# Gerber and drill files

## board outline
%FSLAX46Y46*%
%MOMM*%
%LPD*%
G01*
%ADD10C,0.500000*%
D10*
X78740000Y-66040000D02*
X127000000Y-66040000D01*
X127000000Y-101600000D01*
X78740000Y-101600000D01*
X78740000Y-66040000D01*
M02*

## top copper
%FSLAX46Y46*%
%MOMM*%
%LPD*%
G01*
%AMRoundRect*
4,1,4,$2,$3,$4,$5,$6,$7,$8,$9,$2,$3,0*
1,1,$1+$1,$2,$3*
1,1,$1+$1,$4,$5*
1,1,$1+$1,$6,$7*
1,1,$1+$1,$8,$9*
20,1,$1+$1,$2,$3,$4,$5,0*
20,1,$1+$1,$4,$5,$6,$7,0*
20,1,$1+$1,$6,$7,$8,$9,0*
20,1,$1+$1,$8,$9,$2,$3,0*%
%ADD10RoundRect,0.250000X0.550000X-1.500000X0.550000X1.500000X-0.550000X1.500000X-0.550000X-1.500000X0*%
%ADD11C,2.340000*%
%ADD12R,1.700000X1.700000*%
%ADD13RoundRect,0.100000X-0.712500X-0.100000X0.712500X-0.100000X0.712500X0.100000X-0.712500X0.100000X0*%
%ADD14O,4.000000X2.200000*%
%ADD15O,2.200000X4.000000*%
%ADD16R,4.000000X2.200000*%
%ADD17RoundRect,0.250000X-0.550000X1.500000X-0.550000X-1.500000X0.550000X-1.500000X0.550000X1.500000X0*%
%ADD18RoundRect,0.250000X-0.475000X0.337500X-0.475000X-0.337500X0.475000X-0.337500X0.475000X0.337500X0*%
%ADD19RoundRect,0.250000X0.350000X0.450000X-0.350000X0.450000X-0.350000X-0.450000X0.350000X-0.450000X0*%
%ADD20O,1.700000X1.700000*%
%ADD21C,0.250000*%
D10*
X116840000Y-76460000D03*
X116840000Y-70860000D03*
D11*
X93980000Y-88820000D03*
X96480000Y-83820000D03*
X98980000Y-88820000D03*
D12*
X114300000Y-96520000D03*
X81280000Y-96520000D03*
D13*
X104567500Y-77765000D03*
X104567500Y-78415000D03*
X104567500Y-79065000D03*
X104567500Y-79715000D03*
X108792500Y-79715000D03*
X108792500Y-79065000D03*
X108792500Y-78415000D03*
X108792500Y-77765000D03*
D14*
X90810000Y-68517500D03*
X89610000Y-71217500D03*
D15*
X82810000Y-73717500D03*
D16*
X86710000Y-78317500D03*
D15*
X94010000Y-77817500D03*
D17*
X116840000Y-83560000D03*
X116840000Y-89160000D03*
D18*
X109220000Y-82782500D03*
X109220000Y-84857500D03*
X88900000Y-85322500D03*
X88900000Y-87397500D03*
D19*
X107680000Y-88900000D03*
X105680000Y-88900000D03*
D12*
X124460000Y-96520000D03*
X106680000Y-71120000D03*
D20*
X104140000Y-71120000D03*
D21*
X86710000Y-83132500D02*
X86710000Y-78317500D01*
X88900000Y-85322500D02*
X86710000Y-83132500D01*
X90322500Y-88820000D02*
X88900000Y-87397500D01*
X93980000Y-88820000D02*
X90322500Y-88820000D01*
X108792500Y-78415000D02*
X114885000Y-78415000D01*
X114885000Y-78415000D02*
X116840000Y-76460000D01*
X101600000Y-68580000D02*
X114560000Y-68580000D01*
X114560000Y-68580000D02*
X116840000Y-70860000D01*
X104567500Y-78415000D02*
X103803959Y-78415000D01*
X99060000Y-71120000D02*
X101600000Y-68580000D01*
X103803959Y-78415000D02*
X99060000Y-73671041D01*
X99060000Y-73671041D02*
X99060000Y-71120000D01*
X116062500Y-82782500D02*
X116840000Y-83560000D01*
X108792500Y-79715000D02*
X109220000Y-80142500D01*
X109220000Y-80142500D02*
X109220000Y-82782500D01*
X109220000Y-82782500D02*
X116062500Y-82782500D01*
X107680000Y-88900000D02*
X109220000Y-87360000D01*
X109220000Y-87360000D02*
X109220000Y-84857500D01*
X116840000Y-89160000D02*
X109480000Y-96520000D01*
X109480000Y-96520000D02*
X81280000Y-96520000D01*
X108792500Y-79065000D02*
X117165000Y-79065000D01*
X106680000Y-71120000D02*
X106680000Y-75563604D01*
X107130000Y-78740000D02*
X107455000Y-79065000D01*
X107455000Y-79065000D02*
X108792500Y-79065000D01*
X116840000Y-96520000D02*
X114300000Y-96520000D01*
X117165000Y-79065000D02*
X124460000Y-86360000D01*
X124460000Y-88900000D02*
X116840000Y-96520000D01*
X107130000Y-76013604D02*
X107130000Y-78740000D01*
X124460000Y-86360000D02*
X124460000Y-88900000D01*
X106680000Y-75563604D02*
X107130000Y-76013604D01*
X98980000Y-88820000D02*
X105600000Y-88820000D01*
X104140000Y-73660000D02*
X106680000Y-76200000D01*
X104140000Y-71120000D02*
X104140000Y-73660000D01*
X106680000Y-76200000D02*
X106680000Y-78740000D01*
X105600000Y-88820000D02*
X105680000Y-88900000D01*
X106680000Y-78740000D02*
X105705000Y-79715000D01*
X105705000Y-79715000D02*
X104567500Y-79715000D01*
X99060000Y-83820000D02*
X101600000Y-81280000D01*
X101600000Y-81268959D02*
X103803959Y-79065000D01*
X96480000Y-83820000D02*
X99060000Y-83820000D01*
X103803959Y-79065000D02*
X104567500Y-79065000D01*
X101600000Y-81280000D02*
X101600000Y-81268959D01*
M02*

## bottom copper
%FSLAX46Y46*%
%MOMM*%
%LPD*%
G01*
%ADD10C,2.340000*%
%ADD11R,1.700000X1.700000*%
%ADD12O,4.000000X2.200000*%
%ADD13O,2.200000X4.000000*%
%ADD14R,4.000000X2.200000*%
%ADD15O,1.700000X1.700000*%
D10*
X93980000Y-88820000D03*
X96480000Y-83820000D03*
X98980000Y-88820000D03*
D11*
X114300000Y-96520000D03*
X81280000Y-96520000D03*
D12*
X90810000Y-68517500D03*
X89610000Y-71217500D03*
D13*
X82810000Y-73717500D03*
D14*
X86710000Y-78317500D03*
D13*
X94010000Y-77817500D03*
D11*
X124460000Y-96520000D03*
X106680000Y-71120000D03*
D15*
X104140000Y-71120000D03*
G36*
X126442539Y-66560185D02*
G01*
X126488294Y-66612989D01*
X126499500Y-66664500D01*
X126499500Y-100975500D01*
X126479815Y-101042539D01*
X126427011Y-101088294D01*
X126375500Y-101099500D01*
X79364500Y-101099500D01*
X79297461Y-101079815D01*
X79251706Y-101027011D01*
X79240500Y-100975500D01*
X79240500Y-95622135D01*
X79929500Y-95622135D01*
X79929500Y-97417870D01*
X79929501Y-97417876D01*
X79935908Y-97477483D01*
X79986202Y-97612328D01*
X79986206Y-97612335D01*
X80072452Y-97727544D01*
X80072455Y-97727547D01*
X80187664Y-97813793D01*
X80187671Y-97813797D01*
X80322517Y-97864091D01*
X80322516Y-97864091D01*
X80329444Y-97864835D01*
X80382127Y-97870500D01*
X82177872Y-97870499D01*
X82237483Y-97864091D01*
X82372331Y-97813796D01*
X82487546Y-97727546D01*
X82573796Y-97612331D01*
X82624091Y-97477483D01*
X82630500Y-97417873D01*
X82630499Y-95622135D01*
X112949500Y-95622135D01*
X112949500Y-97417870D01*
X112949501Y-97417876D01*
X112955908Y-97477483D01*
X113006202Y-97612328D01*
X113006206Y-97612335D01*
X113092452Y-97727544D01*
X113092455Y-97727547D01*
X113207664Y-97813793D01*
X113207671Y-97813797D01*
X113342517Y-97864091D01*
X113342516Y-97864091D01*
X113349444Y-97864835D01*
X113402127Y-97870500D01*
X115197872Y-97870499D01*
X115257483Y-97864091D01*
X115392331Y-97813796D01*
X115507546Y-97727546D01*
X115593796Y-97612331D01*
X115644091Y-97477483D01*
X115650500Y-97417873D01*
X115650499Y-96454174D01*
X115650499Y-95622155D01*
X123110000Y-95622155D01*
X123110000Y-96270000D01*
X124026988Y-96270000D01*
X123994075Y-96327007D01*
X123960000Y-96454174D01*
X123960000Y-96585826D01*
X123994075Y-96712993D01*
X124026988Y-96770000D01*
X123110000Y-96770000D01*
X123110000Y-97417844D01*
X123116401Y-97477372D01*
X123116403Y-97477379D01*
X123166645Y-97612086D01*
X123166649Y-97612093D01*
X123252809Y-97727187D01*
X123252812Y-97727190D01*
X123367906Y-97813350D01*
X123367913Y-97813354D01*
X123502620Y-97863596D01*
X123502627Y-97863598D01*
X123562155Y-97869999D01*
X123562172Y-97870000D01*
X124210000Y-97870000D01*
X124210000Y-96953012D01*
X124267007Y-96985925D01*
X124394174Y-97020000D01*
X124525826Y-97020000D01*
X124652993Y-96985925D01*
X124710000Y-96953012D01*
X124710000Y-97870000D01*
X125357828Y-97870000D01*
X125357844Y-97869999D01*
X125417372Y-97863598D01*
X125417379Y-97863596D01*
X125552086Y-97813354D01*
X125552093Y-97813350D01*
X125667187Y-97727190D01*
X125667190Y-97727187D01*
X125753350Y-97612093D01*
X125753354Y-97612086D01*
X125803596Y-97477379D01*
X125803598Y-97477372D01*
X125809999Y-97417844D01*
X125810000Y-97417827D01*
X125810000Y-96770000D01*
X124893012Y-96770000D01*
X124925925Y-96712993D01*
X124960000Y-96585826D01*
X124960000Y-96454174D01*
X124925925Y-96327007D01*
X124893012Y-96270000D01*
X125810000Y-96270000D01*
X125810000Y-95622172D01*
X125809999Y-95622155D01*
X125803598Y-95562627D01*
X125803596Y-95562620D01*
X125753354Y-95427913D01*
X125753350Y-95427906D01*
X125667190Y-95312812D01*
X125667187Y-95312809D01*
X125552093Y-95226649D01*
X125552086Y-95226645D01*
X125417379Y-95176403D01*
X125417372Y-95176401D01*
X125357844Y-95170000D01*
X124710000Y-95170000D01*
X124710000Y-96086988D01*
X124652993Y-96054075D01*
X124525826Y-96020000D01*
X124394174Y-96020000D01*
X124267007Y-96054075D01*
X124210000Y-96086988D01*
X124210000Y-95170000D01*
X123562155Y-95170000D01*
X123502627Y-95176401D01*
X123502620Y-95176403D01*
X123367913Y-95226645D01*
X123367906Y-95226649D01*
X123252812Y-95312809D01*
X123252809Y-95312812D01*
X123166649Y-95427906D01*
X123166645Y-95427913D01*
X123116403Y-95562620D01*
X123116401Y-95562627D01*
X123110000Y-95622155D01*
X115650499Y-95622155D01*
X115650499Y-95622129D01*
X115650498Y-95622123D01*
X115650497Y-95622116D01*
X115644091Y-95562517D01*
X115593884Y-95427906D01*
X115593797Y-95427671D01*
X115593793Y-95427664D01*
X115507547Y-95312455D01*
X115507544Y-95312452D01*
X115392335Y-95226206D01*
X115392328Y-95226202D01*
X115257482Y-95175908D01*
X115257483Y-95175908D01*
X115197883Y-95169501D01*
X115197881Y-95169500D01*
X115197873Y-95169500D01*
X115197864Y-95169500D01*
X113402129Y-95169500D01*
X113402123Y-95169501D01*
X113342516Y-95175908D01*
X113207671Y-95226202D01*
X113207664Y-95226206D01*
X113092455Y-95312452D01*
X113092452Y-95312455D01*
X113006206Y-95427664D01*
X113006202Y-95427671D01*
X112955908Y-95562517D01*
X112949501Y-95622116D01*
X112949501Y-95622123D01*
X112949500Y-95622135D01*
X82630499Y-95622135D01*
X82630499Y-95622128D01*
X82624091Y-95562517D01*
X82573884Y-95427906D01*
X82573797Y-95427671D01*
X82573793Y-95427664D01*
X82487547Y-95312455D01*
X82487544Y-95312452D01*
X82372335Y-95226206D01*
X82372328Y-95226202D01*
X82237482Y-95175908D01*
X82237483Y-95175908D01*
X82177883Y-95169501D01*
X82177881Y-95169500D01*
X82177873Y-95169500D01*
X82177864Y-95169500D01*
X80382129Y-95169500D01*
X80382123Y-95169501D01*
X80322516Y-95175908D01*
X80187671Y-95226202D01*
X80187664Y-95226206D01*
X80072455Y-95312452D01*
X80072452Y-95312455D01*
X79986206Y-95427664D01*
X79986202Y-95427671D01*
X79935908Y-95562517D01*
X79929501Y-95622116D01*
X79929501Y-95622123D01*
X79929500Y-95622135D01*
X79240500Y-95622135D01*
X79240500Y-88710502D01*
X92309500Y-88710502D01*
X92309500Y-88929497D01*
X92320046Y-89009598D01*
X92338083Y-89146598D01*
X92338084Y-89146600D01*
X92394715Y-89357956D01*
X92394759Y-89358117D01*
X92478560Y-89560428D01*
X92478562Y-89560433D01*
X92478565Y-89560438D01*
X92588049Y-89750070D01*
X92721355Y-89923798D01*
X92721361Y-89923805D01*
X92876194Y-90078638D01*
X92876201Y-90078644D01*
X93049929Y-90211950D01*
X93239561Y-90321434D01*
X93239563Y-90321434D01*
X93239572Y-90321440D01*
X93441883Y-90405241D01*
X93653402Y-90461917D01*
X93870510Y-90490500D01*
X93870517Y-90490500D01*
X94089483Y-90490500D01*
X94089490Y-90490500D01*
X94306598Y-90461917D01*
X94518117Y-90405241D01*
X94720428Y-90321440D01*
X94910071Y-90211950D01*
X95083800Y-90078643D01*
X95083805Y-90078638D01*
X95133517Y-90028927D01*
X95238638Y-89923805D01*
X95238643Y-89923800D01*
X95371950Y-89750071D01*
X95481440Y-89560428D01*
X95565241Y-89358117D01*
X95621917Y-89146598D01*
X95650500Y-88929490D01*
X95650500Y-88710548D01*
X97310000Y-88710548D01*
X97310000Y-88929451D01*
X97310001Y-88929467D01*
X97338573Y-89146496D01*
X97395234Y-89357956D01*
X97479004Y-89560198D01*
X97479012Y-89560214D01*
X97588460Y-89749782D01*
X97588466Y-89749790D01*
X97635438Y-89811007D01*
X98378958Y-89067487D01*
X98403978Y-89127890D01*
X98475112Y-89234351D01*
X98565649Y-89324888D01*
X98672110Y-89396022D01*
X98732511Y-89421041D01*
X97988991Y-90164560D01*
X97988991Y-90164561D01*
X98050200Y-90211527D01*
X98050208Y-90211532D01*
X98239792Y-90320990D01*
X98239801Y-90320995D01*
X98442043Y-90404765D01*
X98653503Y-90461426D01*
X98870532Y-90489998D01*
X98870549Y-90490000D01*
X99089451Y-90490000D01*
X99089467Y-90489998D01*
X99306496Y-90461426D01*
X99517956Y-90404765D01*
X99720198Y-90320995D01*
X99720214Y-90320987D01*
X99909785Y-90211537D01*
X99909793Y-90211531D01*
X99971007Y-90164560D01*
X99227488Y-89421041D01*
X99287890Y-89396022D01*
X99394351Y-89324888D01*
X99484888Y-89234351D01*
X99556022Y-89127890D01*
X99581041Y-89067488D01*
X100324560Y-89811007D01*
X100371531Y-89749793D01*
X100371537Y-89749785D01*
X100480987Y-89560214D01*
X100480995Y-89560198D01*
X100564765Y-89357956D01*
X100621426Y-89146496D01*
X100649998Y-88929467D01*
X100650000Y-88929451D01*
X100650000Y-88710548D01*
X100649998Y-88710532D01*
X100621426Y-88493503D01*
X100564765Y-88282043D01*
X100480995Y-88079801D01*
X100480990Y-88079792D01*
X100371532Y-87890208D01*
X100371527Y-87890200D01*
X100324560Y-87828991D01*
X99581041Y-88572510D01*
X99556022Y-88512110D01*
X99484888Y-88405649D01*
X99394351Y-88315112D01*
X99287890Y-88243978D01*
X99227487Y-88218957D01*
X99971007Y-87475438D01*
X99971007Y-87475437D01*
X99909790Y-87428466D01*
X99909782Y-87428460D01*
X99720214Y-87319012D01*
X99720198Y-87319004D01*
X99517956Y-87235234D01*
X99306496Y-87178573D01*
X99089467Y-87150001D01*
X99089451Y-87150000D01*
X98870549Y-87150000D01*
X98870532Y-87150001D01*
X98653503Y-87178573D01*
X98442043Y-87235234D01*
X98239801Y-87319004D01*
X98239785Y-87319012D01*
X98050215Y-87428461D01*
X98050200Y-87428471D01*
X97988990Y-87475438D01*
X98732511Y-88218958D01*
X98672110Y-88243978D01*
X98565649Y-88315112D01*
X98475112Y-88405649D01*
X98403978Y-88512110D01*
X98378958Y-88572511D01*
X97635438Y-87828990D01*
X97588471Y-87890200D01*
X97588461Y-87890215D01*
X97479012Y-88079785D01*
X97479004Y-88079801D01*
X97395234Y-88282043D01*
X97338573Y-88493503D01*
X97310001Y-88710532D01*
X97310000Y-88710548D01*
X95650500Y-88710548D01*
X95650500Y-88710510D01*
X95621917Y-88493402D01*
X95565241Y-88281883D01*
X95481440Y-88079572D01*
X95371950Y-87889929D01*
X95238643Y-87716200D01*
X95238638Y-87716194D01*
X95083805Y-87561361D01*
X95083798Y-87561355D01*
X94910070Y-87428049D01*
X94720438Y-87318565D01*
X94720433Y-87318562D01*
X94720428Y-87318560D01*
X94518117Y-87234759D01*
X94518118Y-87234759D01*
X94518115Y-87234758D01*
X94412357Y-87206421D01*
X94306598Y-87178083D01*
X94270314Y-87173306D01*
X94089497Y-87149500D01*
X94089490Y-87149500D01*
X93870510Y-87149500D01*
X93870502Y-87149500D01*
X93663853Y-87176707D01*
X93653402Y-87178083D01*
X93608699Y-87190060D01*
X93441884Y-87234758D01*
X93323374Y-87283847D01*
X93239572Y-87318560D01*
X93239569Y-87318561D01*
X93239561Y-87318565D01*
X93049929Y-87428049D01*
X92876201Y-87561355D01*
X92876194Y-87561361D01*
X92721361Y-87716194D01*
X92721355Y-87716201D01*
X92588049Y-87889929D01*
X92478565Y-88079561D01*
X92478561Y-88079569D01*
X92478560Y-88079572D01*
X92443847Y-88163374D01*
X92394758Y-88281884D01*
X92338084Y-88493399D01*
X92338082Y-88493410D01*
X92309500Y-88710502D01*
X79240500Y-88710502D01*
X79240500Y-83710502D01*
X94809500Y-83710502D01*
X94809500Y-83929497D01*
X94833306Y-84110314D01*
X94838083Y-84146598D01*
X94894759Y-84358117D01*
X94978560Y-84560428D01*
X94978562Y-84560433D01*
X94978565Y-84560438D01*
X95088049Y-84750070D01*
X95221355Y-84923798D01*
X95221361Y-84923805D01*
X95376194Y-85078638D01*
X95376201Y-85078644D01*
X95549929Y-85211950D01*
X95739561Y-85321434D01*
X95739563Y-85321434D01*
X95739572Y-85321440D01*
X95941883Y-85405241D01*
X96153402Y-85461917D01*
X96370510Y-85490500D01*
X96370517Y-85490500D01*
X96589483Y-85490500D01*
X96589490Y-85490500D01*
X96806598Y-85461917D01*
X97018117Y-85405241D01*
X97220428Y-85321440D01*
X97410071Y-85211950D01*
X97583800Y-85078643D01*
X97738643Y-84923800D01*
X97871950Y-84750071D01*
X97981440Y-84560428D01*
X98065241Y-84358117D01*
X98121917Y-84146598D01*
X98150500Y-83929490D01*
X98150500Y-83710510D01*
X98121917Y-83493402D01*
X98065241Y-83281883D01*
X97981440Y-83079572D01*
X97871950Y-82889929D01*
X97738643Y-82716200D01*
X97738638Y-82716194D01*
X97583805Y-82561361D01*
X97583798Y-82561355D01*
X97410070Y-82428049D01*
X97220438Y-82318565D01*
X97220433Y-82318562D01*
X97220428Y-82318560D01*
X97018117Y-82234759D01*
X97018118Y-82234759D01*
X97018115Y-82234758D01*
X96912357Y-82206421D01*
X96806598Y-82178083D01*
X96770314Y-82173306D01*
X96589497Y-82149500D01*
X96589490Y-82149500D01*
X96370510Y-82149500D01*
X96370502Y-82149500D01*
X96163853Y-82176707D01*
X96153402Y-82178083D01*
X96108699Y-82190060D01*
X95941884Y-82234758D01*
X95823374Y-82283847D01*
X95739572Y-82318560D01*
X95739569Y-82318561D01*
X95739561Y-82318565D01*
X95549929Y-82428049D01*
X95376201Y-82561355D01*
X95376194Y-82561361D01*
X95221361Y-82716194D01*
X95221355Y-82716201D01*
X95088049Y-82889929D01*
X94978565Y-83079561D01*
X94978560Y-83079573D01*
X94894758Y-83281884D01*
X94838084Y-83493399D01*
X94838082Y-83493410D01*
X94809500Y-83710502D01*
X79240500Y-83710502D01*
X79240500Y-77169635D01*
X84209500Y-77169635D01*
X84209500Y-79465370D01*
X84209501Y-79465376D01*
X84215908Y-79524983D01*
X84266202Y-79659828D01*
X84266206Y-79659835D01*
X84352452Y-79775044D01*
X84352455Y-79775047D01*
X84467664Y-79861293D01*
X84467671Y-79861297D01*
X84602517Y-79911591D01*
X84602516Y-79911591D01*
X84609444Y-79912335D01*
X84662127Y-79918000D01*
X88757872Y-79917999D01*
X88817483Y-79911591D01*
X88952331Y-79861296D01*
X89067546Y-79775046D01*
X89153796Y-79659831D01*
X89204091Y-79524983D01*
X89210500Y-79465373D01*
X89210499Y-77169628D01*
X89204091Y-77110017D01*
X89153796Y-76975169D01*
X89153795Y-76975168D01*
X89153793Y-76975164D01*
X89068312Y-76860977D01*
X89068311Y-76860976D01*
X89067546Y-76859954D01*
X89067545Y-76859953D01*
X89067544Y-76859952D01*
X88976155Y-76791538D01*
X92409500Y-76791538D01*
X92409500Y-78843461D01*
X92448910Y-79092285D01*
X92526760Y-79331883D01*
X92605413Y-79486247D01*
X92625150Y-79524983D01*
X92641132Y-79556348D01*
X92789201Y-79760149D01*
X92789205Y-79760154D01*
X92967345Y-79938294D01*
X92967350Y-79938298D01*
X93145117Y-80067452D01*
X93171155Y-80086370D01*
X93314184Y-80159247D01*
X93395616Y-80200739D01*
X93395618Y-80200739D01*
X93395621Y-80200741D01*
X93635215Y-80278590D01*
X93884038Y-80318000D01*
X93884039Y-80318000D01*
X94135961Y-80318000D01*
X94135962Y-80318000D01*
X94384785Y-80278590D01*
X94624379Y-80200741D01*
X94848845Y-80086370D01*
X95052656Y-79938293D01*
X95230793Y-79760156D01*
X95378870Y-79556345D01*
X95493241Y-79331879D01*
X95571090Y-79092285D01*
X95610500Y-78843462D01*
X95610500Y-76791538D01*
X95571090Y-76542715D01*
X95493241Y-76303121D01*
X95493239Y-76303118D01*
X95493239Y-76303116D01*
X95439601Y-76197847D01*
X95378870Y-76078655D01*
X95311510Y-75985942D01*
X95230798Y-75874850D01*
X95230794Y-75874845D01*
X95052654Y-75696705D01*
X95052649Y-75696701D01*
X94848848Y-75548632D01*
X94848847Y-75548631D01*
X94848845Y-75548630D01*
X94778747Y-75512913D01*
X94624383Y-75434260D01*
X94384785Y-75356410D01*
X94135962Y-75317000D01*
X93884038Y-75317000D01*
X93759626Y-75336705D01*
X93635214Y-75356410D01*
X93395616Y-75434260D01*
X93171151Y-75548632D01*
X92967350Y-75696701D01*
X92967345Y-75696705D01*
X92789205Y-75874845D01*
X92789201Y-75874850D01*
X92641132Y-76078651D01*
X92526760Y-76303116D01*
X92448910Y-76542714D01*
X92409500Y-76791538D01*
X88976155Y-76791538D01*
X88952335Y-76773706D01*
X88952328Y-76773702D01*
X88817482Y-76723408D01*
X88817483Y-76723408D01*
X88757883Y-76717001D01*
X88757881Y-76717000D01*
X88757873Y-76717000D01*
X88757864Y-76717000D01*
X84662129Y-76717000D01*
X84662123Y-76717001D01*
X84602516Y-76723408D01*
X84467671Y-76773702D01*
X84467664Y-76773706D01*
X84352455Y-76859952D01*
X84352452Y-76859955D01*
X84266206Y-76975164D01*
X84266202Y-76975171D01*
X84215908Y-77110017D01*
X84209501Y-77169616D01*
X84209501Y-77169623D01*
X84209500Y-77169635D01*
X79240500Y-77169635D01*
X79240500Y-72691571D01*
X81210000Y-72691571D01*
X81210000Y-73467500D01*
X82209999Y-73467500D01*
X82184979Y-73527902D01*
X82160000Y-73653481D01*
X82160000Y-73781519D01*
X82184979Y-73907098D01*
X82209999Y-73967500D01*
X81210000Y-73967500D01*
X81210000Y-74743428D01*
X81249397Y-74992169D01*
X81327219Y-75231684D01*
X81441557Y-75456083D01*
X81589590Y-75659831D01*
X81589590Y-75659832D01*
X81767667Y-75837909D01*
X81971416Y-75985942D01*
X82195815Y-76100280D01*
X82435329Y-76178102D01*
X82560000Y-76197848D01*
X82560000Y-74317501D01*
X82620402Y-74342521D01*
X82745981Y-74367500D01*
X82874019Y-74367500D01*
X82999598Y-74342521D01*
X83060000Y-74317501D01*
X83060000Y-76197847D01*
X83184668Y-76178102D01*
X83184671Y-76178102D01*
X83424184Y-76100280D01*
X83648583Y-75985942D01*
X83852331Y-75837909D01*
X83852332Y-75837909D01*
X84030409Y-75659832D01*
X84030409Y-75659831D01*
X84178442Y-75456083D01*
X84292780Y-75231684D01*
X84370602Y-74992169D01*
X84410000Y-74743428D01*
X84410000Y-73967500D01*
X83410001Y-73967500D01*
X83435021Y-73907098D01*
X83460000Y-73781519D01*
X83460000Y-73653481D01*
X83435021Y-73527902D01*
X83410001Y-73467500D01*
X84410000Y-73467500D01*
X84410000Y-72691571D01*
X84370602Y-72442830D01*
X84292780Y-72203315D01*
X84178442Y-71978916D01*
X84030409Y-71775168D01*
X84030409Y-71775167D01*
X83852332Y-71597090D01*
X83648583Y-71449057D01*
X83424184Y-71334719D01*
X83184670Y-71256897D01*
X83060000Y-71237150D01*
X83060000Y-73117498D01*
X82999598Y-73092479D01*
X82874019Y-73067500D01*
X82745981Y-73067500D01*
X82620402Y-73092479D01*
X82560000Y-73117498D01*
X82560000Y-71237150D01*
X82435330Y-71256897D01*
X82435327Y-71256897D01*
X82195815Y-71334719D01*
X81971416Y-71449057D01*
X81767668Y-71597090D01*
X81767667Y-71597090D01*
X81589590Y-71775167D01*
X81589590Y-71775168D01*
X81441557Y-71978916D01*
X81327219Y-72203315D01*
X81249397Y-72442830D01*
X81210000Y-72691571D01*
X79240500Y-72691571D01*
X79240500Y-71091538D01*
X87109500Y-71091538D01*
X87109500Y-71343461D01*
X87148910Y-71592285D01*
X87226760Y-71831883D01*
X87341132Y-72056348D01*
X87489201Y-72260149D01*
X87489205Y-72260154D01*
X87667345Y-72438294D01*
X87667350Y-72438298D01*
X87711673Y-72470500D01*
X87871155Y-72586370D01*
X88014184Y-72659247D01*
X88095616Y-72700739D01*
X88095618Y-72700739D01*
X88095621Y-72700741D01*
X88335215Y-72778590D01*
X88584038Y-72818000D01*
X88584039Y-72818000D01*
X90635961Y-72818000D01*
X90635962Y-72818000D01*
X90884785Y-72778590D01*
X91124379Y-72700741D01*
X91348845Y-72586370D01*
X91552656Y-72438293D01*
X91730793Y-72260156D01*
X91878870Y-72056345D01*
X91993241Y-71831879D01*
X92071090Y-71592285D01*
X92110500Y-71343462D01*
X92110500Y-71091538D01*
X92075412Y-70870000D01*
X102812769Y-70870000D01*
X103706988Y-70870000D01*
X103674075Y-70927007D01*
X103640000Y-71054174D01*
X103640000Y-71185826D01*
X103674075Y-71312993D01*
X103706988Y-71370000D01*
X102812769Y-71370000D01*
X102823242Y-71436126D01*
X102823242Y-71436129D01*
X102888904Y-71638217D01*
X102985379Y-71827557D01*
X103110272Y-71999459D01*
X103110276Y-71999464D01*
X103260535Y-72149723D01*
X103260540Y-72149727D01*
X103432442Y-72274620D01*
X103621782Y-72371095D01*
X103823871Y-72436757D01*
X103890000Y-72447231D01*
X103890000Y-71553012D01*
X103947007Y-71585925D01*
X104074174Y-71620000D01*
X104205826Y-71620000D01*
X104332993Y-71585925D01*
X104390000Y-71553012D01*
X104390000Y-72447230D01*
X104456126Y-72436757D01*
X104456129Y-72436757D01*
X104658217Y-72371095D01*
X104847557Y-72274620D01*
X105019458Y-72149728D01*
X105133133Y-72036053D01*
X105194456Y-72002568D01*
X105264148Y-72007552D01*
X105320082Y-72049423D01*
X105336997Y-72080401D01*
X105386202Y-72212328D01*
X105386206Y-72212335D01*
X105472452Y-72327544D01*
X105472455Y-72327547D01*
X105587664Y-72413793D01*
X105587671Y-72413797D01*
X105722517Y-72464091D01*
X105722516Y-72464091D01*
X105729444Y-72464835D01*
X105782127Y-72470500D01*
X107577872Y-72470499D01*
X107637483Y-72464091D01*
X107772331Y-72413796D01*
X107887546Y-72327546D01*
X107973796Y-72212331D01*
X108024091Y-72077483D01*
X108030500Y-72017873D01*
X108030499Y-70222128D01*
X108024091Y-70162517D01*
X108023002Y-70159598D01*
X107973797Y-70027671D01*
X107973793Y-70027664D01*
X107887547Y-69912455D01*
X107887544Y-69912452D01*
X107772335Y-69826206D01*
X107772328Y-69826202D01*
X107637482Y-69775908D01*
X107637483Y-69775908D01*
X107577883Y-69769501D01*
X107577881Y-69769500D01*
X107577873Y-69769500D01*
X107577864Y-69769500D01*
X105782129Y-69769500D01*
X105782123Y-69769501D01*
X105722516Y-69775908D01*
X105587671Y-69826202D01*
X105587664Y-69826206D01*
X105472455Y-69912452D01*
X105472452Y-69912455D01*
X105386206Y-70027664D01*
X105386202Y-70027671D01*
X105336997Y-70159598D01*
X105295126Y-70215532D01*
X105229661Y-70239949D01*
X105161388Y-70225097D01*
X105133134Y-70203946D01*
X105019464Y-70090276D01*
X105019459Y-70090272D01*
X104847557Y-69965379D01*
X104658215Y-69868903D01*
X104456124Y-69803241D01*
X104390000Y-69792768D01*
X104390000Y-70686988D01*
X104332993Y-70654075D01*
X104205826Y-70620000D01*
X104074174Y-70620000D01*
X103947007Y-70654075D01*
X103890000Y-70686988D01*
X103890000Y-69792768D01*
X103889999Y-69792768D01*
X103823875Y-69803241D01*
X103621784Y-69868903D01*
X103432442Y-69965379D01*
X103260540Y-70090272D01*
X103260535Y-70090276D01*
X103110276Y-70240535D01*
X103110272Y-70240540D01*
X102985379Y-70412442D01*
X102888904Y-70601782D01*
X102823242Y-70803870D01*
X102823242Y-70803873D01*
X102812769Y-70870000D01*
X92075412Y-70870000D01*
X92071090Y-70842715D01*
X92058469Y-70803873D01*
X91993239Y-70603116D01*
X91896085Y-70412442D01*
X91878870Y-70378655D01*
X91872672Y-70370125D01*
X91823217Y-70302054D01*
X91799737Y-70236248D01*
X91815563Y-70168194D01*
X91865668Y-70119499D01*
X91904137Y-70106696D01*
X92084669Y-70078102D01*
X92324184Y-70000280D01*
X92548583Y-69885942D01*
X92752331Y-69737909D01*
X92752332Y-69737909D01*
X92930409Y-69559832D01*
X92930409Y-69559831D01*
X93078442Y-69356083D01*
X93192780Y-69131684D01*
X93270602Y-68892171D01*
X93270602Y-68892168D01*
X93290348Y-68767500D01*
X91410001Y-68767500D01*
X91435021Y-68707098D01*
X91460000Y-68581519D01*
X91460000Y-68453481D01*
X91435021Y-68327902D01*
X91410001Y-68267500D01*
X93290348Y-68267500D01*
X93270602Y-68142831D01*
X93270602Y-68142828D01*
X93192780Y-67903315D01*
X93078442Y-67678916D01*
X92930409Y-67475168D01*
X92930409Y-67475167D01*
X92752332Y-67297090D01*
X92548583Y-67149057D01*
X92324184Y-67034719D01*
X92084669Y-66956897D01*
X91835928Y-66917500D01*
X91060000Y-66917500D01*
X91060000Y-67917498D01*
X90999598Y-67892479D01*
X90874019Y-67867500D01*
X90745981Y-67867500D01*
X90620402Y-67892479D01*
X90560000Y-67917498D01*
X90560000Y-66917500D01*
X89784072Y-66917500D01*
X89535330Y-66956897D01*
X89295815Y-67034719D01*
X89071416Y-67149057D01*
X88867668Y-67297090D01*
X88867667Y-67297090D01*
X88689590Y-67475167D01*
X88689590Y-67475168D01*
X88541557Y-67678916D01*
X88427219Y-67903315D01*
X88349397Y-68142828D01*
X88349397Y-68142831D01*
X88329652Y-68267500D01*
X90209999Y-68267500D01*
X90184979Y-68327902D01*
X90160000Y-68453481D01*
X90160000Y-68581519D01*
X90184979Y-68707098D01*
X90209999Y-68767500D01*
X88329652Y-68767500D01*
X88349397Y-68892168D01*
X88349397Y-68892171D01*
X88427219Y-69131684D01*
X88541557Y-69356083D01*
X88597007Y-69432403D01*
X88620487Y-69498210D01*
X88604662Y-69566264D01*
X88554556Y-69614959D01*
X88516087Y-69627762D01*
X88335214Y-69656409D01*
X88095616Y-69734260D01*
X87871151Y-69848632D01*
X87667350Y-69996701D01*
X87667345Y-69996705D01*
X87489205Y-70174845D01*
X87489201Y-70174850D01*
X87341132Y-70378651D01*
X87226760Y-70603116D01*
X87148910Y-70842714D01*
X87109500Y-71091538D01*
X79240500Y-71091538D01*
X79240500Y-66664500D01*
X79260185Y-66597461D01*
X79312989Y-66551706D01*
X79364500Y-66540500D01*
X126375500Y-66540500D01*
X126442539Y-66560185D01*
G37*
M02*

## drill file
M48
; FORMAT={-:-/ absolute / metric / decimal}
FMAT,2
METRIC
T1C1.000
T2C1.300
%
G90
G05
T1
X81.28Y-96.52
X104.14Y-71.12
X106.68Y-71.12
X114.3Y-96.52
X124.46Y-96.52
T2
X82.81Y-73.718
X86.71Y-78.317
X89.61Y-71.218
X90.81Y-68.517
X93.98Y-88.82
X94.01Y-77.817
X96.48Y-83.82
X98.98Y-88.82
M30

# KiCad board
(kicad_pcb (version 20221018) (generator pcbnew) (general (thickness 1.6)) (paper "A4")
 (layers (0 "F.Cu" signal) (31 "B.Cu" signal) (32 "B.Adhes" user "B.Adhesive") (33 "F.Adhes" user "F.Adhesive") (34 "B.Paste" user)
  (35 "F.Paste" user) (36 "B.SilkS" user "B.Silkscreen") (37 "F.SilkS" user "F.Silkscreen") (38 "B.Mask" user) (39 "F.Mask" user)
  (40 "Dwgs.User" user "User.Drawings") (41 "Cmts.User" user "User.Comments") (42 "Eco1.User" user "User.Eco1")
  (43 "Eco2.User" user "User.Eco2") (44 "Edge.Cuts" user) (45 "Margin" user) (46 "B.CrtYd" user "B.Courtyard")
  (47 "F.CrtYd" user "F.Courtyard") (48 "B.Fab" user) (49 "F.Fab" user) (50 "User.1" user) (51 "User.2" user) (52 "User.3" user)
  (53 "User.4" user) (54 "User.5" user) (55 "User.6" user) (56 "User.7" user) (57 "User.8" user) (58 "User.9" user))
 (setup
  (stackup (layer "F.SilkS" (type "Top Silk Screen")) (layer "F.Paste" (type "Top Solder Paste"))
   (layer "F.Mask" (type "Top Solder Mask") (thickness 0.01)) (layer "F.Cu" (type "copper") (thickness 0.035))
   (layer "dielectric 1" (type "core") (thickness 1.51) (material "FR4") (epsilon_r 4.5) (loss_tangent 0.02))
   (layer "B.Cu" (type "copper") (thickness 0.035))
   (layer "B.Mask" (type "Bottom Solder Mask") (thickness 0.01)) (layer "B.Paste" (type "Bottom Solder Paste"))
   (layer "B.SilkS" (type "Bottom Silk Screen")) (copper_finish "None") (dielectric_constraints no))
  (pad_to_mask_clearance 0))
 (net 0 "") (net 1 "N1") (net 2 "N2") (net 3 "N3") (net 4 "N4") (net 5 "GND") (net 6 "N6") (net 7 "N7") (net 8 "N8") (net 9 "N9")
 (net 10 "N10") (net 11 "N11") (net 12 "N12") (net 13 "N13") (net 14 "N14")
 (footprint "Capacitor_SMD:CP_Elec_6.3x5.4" (layer "F.Cu") (at 116.84 73.66 90)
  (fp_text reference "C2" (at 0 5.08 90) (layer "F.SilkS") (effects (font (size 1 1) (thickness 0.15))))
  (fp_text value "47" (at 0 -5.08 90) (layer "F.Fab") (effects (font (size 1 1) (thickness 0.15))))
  (pad "1" smd roundrect (at -2.8 0 90) (size 3.5 1.6) (layers "F.Cu" "F.Paste" "F.Mask") (roundrect_rratio 0.15625) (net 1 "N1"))
  (pad "2" smd roundrect (at 2.8 0 90) (size 3.5 1.6) (layers "F.Cu" "F.Paste" "F.Mask") (roundrect_rratio 0.15625) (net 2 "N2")))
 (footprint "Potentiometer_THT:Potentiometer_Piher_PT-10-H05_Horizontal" (layer "F.Cu") (at 93.98 88.82 90)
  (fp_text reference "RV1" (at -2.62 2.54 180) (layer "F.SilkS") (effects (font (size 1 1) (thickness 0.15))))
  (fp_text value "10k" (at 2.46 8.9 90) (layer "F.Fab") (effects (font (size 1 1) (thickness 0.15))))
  (pad "1" thru_hole circle (at 0 0 90) (size 2.34 2.34) (drill 1.3) (layers "*.Cu" "*.Mask") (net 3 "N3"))
  (pad "2" thru_hole circle (at 5 2.5 90) (size 2.34 2.34) (drill 1.3) (layers "*.Cu" "*.Mask") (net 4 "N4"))
  (pad "3" thru_hole circle (at 0 5 90) (size 2.34 2.34) (drill 1.3) (layers "*.Cu" "*.Mask") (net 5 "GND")))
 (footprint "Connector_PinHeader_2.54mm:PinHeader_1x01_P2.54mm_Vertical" (layer "F.Cu") (at 114.3 96.52)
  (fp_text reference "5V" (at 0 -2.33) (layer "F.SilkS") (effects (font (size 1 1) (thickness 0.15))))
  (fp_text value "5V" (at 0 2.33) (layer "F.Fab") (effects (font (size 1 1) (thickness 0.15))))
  (pad "1" thru_hole rect (at 0 0) (size 1.7 1.7) (drill 1) (layers "*.Cu" "*.Mask") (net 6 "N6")))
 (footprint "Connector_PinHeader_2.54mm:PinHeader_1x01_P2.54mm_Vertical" (layer "F.Cu") (at 81.28 96.52)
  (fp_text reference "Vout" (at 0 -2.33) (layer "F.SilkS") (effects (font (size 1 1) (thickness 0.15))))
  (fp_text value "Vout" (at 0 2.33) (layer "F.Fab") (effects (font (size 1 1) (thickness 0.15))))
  (pad "1" thru_hole rect (at 0 0) (size 1.7 1.7) (drill 1) (layers "*.Cu" "*.Mask") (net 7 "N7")))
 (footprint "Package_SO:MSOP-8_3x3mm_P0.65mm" (layer "F.Cu") (at 106.68 78.74)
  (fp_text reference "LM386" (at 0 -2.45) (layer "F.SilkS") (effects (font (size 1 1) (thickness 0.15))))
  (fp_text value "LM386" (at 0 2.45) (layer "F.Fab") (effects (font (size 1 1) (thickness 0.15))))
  (pad "1" smd roundrect (at -2.1125 -0.975) (size 1.625 0.4) (layers "F.Cu" "F.Paste" "F.Mask") (roundrect_rratio 0.25) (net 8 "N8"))
  (pad "2" smd roundrect (at -2.1125 -0.325) (size 1.625 0.4) (layers "F.Cu" "F.Paste" "F.Mask") (roundrect_rratio 0.25) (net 2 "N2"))
  (pad "3" smd roundrect (at -2.1125 0.325) (size 1.625 0.4) (layers "F.Cu" "F.Paste" "F.Mask") (roundrect_rratio 0.25) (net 4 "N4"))
  (pad "4" smd roundrect (at -2.1125 0.975) (size 1.625 0.4) (layers "F.Cu" "F.Paste" "F.Mask") (roundrect_rratio 0.25) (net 5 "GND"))
  (pad "5" smd roundrect (at 2.1125 0.975) (size 1.625 0.4) (layers "F.Cu" "F.Paste" "F.Mask") (roundrect_rratio 0.25) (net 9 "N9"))
  (pad "6" smd roundrect (at 2.1125 0.325) (size 1.625 0.4) (layers "F.Cu" "F.Paste" "F.Mask") (roundrect_rratio 0.25) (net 6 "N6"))
  (pad "7" smd roundrect (at 2.1125 -0.325) (size 1.625 0.4) (layers "F.Cu" "F.Paste" "F.Mask") (roundrect_rratio 0.25) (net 1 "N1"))
  (pad "8" smd roundrect (at 2.1125 -0.975) (size 1.625 0.4) (layers "F.Cu" "F.Paste" "F.Mask") (roundrect_rratio 0.25) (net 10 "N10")))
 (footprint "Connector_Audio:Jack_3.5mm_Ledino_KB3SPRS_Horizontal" (layer "F.Cu") (at 86.71 78.3175)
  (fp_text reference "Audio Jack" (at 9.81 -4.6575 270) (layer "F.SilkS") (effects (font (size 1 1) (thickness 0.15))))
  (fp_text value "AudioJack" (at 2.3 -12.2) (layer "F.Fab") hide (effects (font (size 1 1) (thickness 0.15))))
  (pad "R" thru_hole oval (at 4.1 -9.8) (size 4 2.2) (drill 1.3) (layers "*.Cu" "*.Mask") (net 5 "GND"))
  (pad "RN" thru_hole oval (at 2.9 -7.1) (size 4 2.2) (drill 1.3) (layers "*.Cu" "*.Mask") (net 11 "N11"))
  (pad "S" thru_hole oval (at -3.9 -4.6) (size 2.2 4) (drill 1.3) (layers "*.Cu" "*.Mask") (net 5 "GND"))
  (pad "T" thru_hole rect (at 0 0) (size 4 2.2) (drill 1.3) (layers "*.Cu" "*.Mask") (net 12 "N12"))
  (pad "TN" thru_hole oval (at 7.3 -0.5 90) (size 4 2.2) (drill 1.3) (layers "*.Cu" "*.Mask") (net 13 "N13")))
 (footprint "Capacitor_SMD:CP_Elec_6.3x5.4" (layer "F.Cu") (at 116.84 86.36 -90)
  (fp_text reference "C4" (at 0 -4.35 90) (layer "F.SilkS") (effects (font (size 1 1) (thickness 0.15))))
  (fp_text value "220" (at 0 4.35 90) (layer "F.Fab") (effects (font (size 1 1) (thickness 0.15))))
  (pad "1" smd roundrect (at -2.8 0 270) (size 3.5 1.6) (layers "F.Cu" "F.Paste" "F.Mask") (roundrect_rratio 0.15625) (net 9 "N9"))
  (pad "2" smd roundrect (at 2.8 0 270) (size 3.5 1.6) (layers "F.Cu" "F.Paste" "F.Mask") (roundrect_rratio 0.15625) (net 7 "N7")))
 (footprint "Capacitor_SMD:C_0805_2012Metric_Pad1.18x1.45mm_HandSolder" (layer "F.Cu") (at 109.22 83.82 -90)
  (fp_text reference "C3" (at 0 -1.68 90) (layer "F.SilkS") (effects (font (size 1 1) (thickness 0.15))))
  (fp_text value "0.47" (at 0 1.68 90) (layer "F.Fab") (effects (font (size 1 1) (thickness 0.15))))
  (pad "1" smd roundrect (at -1.0375 0 270) (size 1.175 1.45) (layers "F.Cu" "F.Paste" "F.Mask") (roundrect_rratio 0.2127659574)
   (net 9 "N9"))
  (pad "2" smd roundrect (at 1.0375 0 270) (size 1.175 1.45) (layers "F.Cu" "F.Paste" "F.Mask") (roundrect_rratio 0.2127659574)
   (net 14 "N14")))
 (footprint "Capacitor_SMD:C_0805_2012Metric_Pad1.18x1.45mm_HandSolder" (layer "F.Cu") (at 88.9 86.36 -90)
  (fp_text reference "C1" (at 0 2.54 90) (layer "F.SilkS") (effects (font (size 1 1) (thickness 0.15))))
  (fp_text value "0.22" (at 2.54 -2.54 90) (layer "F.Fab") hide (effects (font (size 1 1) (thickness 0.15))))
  (pad "1" smd roundrect (at -1.0375 0 270) (size 1.175 1.45) (layers "F.Cu" "F.Paste" "F.Mask") (roundrect_rratio 0.2127659574)
   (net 12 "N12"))
  (pad "2" smd roundrect (at 1.0375 0 270) (size 1.175 1.45) (layers "F.Cu" "F.Paste" "F.Mask") (roundrect_rratio 0.2127659574) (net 3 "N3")))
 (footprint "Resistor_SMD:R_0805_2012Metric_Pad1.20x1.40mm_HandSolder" (layer "F.Cu") (at 106.68 88.9 180)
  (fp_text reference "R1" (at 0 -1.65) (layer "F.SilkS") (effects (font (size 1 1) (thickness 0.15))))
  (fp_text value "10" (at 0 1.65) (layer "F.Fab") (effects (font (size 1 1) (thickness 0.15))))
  (pad "1" smd roundrect (at -1 0 180) (size 1.2 1.4) (layers "F.Cu" "F.Paste" "F.Mask") (roundrect_rratio 0.2083333333) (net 14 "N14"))
  (pad "2" smd roundrect (at 1 0 180) (size 1.2 1.4) (layers "F.Cu" "F.Paste" "F.Mask") (roundrect_rratio 0.2083333333) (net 5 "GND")))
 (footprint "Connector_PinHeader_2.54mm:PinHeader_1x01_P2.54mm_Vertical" (layer "F.Cu") (at 124.46 96.52)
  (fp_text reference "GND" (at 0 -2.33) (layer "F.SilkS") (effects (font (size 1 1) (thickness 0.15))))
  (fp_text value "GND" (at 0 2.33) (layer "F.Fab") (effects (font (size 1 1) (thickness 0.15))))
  (pad "1" thru_hole rect (at 0 0) (size 1.7 1.7) (drill 1) (layers "*.Cu" "*.Mask") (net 5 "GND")))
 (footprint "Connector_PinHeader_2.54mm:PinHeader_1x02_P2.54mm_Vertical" (layer "F.Cu") (at 106.68 71.12 -90)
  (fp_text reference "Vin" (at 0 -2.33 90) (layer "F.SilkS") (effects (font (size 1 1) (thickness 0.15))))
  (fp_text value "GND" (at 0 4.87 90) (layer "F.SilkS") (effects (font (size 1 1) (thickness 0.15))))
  (pad "1" thru_hole rect (at 0 0 270) (size 1.7 1.7) (drill 1) (layers "*.Cu" "*.Mask") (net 6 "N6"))
  (pad "2" thru_hole oval (at 0 2.54 270) (size 1.7 1.7) (drill 1) (layers "*.Cu" "*.Mask") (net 5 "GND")))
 (gr_rect (start 78.74 66.04) (end 127 101.6) (stroke (width 0.5) (type default)) (fill none) (layer "Edge.Cuts"))
 (segment (start 86.71 83.1325) (end 86.71 78.3175) (width 0.25) (layer "F.Cu") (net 12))
 (segment (start 88.9 85.3225) (end 86.71 83.1325) (width 0.25) (layer "F.Cu") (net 12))
 (segment (start 90.3225 88.82) (end 88.9 87.3975) (width 0.25) (layer "F.Cu") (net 3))
 (segment (start 93.98 88.82) (end 90.3225 88.82) (width 0.25) (layer "F.Cu") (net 3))
 (segment (start 108.7925 78.415) (end 114.885 78.415) (width 0.25) (layer "F.Cu") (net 1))
 (segment (start 114.885 78.415) (end 116.84 76.46) (width 0.25) (layer "F.Cu") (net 1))
 (segment (start 101.6 68.58) (end 114.56 68.58) (width 0.25) (layer "F.Cu") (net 2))
 (segment (start 114.56 68.58) (end 116.84 70.86) (width 0.25) (layer "F.Cu") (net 2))
 (segment (start 104.5675 78.415) (end 103.803959 78.415) (width 0.25) (layer "F.Cu") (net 2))
 (segment (start 99.06 71.12) (end 101.6 68.58) (width 0.25) (layer "F.Cu") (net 2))
 (segment (start 103.803959 78.415) (end 99.06 73.671041) (width 0.25) (layer "F.Cu") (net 2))
 (segment (start 99.06 73.671041) (end 99.06 71.12) (width 0.25) (layer "F.Cu") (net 2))
 (segment (start 116.0625 82.7825) (end 116.84 83.56) (width 0.25) (layer "F.Cu") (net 9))
 (segment (start 108.7925 79.715) (end 109.22 80.1425) (width 0.25) (layer "F.Cu") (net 9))
 (segment (start 109.22 80.1425) (end 109.22 82.7825) (width 0.25) (layer "F.Cu") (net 9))
 (segment (start 109.22 82.7825) (end 116.0625 82.7825) (width 0.25) (layer "F.Cu") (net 9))
 (segment (start 107.68 88.9) (end 109.22 87.36) (width 0.25) (layer "F.Cu") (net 14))
 (segment (start 109.22 87.36) (end 109.22 84.8575) (width 0.25) (layer "F.Cu") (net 14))
 (segment (start 116.84 89.16) (end 109.48 96.52) (width 0.25) (layer "F.Cu") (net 7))
 (segment (start 109.48 96.52) (end 81.28 96.52) (width 0.25) (layer "F.Cu") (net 7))
 (segment (start 108.7925 79.065) (end 117.165 79.065) (width 0.25) (layer "F.Cu") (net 6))
 (segment (start 106.68 71.12) (end 106.68 75.563604) (width 0.25) (layer "F.Cu") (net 6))
 (segment (start 107.13 78.74) (end 107.455 79.065) (width 0.25) (layer "F.Cu") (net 6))
 (segment (start 107.455 79.065) (end 108.7925 79.065) (width 0.25) (layer "F.Cu") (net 6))
 (segment (start 116.84 96.52) (end 114.3 96.52) (width 0.25) (layer "F.Cu") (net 6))
 (segment (start 117.165 79.065) (end 124.46 86.36) (width 0.25) (layer "F.Cu") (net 6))
 (segment (start 124.46 88.9) (end 116.84 96.52) (width 0.25) (layer "F.Cu") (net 6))
 (segment (start 107.13 76.013604) (end 107.13 78.74) (width 0.25) (layer "F.Cu") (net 6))
 (segment (start 124.46 86.36) (end 124.46 88.9) (width 0.25) (layer "F.Cu") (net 6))
 (segment (start 106.68 75.563604) (end 107.13 76.013604) (width 0.25) (layer "F.Cu") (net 6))
 (segment (start 98.98 88.82) (end 105.6 88.82) (width 0.25) (layer "F.Cu") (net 5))
 (segment (start 104.14 73.66) (end 106.68 76.2) (width 0.25) (layer "F.Cu") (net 5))
 (segment (start 104.14 71.12) (end 104.14 73.66) (width 0.25) (layer "F.Cu") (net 5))
 (segment (start 106.68 76.2) (end 106.68 78.74) (width 0.25) (layer "F.Cu") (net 5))
 (segment (start 105.6 88.82) (end 105.68 88.9) (width 0.25) (layer "F.Cu") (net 5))
 (segment (start 106.68 78.74) (end 105.705 79.715) (width 0.25) (layer "F.Cu") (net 5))
 (segment (start 105.705 79.715) (end 104.5675 79.715) (width 0.25) (layer "F.Cu") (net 5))
 (segment (start 99.06 83.82) (end 101.6 81.28) (width 0.25) (layer "F.Cu") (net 4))
 (segment (start 101.6 81.268959) (end 103.803959 79.065) (width 0.25) (layer "F.Cu") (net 4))
 (segment (start 96.48 83.82) (end 99.06 83.82) (width 0.25) (layer "F.Cu") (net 4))
 (segment (start 103.803959 79.065) (end 104.5675 79.065) (width 0.25) (layer "F.Cu") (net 4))
 (segment (start 101.6 81.28) (end 101.6 81.268959) (width 0.25) (layer "F.Cu") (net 4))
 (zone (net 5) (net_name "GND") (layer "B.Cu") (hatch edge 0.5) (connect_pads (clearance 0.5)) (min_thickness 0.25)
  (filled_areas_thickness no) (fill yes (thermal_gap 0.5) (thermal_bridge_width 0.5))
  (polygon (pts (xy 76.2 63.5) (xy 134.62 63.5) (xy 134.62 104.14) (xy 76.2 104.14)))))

